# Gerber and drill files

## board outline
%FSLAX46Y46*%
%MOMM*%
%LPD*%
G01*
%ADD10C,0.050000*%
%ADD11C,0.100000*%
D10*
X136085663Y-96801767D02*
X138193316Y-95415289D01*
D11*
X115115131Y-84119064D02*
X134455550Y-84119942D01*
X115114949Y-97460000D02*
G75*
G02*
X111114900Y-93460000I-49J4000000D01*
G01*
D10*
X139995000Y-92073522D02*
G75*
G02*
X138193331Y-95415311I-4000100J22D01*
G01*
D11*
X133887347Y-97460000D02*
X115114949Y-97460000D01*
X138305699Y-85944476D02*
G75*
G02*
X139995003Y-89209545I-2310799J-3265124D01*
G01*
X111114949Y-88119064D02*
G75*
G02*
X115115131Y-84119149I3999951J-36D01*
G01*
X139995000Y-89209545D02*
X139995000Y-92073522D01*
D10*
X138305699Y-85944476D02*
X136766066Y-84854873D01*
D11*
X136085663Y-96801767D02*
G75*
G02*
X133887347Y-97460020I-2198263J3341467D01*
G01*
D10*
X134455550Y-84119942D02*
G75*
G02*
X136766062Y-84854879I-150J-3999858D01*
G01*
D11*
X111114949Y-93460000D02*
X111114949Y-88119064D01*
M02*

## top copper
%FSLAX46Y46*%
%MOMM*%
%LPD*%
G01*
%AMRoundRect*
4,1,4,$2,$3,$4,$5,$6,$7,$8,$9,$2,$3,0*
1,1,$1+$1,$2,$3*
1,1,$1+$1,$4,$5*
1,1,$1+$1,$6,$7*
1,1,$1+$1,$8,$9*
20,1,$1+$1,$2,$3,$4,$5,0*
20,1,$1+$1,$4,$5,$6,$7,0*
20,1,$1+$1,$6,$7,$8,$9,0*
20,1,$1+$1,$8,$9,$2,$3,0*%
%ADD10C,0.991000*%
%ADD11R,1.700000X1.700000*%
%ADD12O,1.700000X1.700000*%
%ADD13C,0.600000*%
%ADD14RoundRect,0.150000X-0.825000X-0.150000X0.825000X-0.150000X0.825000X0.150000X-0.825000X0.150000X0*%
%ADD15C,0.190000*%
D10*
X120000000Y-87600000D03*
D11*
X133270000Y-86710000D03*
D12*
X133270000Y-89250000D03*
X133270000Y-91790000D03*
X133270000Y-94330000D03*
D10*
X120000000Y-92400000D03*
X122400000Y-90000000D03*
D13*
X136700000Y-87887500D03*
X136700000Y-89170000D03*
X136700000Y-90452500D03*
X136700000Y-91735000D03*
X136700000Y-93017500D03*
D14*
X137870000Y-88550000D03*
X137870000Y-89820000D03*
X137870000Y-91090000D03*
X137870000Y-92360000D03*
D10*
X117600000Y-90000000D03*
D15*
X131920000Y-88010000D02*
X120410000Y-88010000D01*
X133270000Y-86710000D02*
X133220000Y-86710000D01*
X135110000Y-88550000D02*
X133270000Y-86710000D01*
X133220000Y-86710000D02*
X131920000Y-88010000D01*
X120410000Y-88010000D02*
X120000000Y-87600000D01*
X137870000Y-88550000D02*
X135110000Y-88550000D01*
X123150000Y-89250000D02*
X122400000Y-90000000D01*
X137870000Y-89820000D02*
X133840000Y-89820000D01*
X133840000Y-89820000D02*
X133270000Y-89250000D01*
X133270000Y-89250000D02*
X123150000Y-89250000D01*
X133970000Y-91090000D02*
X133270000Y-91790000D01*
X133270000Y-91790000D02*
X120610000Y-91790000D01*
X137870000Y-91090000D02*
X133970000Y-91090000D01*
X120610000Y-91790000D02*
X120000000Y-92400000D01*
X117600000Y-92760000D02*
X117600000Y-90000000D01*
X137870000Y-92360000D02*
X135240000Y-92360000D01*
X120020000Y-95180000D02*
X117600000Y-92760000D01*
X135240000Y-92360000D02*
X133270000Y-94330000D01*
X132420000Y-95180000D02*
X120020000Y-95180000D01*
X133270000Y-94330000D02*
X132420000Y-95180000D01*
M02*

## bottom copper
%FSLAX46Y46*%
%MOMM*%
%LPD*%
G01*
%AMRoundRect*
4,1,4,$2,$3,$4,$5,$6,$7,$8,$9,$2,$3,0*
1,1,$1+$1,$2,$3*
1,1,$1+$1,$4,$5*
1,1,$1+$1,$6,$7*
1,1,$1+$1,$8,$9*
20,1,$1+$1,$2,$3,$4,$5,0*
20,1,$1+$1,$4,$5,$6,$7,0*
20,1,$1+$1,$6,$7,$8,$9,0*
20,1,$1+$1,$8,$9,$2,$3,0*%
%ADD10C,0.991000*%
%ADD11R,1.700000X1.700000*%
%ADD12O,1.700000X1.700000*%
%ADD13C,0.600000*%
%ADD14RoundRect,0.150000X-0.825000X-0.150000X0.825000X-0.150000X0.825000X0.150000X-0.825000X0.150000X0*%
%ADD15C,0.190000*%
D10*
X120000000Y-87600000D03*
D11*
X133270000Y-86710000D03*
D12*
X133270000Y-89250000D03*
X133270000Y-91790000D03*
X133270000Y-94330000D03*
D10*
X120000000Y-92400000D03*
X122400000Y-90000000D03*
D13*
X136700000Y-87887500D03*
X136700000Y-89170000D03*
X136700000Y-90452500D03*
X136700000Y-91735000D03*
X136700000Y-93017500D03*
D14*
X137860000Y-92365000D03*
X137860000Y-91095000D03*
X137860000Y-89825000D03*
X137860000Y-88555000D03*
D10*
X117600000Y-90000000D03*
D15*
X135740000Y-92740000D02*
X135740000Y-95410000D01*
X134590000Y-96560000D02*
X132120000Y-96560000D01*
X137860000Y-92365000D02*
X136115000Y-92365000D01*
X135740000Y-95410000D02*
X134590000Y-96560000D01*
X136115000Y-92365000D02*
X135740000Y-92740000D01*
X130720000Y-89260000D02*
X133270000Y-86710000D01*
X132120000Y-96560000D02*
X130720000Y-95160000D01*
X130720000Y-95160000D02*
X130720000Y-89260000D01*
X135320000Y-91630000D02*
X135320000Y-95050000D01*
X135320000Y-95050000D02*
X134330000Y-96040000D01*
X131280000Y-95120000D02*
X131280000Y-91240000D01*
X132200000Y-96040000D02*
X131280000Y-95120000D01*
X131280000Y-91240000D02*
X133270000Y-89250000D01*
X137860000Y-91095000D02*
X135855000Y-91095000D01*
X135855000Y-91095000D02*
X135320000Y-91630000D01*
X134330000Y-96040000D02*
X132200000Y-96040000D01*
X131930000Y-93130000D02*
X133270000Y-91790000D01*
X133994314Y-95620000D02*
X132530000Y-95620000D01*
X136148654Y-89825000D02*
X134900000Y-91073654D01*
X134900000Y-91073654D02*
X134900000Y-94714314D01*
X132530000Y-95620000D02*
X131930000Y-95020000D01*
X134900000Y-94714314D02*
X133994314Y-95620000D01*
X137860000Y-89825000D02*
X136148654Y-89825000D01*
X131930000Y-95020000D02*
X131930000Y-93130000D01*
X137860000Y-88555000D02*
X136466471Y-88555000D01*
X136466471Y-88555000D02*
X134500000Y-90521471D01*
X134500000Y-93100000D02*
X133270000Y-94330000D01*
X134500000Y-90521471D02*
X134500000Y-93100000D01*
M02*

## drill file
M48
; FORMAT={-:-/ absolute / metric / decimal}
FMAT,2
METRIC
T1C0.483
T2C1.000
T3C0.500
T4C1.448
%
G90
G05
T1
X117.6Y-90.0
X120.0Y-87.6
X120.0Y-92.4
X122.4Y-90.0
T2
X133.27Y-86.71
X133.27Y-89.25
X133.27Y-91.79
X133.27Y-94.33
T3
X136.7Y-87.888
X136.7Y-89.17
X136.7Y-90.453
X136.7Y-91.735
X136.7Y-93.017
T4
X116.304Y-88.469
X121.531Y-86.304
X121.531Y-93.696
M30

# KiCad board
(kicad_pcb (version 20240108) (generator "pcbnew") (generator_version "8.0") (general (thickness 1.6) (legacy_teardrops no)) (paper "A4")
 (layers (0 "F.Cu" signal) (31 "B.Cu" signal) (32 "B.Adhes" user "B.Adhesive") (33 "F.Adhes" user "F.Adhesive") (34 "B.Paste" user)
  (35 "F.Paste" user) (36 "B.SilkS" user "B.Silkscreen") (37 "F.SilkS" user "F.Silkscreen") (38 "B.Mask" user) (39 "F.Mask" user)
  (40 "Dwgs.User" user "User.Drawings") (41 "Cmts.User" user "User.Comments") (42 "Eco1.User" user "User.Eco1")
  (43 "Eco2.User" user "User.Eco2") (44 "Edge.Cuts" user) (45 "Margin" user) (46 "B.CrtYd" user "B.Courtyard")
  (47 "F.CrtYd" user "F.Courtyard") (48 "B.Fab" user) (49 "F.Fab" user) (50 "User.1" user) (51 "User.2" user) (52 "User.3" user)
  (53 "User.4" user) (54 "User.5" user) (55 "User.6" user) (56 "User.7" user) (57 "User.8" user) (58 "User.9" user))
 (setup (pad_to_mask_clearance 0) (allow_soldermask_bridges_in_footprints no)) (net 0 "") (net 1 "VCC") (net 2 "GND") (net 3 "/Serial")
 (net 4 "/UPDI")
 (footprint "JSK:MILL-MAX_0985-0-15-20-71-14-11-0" (layer "F.Cu") (at 120 87.6)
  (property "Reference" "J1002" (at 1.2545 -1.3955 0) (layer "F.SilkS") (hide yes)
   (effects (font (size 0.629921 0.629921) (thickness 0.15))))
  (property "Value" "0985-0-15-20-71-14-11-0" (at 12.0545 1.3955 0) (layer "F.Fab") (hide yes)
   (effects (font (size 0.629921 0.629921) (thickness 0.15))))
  (pad "1" thru_hole circle (at 0 0) (size 0.991 0.991) (drill 0.483) (layers "*.Cu" "*.Mask") (remove_unused_layers no) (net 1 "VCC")
   (solder_mask_margin 0.102)))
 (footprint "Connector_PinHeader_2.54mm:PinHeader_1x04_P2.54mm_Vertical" (layer "F.Cu") (at 133.27 86.71)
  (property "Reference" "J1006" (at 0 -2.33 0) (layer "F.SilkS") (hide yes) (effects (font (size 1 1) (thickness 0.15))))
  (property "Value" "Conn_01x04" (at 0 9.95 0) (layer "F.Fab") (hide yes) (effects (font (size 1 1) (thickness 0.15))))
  (pad "1" thru_hole rect (at 0 0) (size 1.7 1.7) (drill 1) (layers "*.Cu" "*.Mask") (remove_unused_layers no) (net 1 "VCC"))
  (pad "2" thru_hole oval (at 0 2.54) (size 1.7 1.7) (drill 1) (layers "*.Cu" "*.Mask") (remove_unused_layers no) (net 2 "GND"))
  (pad "3" thru_hole oval (at 0 5.08) (size 1.7 1.7) (drill 1) (layers "*.Cu" "*.Mask") (remove_unused_layers no) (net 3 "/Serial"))
  (pad "4" thru_hole oval (at 0 7.62) (size 1.7 1.7) (drill 1) (layers "*.Cu" "*.Mask") (remove_unused_layers no) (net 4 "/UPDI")))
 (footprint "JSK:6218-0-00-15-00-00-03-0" (layer "F.Cu") (at 121.530733 93.695518)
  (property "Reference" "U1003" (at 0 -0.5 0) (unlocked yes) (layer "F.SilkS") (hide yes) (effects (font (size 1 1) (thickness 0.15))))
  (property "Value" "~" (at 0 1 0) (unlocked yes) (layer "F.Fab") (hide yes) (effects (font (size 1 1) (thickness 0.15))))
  (pad "" np_thru_hole circle (at 0 0) (size 1.648 1.648) (drill 1.448) (layers "*.Mask")))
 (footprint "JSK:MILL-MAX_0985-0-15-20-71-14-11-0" (layer "F.Cu") (at 120 92.4)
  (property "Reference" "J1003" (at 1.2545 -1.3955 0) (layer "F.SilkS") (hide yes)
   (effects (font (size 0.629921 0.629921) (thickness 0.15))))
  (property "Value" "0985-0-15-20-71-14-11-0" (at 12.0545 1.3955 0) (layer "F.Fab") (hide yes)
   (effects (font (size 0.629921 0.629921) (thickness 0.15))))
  (pad "1" thru_hole circle (at 0 0) (size 0.991 0.991) (drill 0.483) (layers "*.Cu" "*.Mask") (remove_unused_layers no) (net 3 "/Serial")
   (solder_mask_margin 0.102)))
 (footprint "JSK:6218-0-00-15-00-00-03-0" (layer "F.Cu") (at 121.530733 86.304481)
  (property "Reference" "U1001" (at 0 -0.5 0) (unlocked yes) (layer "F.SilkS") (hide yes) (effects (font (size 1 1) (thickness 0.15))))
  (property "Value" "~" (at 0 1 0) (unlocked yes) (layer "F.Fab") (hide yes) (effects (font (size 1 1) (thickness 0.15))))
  (pad "" np_thru_hole circle (at 0 0) (size 1.648 1.648) (drill 1.448) (layers "*.Mask")))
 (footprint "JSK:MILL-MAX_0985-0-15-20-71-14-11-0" (layer "F.Cu") (at 122.4 90)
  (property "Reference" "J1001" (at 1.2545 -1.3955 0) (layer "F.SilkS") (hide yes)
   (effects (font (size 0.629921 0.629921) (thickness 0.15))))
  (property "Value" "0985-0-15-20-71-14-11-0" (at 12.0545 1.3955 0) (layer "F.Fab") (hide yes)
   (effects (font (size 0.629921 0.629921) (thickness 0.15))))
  (pad "1" thru_hole circle (at 0 0) (size 0.991 0.991) (drill 0.483) (layers "*.Cu" "*.Mask") (remove_unused_layers no) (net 2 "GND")
   (solder_mask_margin 0.102)))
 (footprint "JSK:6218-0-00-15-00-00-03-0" (layer "F.Cu") (at 116.304481 88.469266)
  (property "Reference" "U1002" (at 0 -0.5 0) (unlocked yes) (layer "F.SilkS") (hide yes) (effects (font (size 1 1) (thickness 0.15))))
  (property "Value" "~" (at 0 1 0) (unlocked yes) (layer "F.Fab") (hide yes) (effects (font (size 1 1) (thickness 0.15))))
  (pad "" np_thru_hole circle (at 0 0) (size 1.648 1.648) (drill 1.448) (layers "*.Mask")))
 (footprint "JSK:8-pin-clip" (layer "F.Cu") (at 137.87 90.455)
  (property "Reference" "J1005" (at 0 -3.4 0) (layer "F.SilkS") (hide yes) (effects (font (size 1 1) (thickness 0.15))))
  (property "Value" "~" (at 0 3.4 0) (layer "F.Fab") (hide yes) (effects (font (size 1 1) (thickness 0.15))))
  (pad "" np_thru_hole circle (at -1.17 -2.5675) (size 0.6 0.6) (drill 0.5) (layers "F&B.Cu"))
  (pad "" np_thru_hole circle (at -1.17 -1.285) (size 0.6 0.6) (drill 0.5) (layers "F&B.Cu"))
  (pad "" np_thru_hole circle (at -1.17 -0.0025) (size 0.6 0.6) (drill 0.5) (layers "F&B.Cu"))
  (pad "" np_thru_hole circle (at -1.17 1.28) (size 0.6 0.6) (drill 0.5) (layers "F&B.Cu"))
  (pad "" np_thru_hole circle (at -1.17 2.5625) (size 0.6 0.6) (drill 0.5) (layers "F&B.Cu"))
  (pad "A1" smd roundrect (at 0 -1.905) (size 1.95 0.6) (layers "F.Cu" "F.Paste" "F.Mask") (roundrect_rratio 0.25) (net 1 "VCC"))
  (pad "A2" smd roundrect (at 0 -0.635) (size 1.95 0.6) (layers "F.Cu" "F.Paste" "F.Mask") (roundrect_rratio 0.25) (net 2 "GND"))
  (pad "A3" smd roundrect (at 0 0.635) (size 1.95 0.6) (layers "F.Cu" "F.Paste" "F.Mask") (roundrect_rratio 0.25) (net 3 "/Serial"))
  (pad "A4" smd roundrect (at 0 1.905) (size 1.95 0.6) (layers "F.Cu" "F.Paste" "F.Mask") (roundrect_rratio 0.25) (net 4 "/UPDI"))
  (pad "B1" smd roundrect (at -0.01 1.91) (size 1.95 0.6) (layers "B.Cu" "B.Paste" "B.Mask") (roundrect_rratio 0.25) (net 1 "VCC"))
  (pad "B2" smd roundrect (at -0.01 0.64) (size 1.95 0.6) (layers "B.Cu" "B.Paste" "B.Mask") (roundrect_rratio 0.25) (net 2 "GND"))
  (pad "B3" smd roundrect (at -0.01 -0.63) (size 1.95 0.6) (layers "B.Cu" "B.Paste" "B.Mask") (roundrect_rratio 0.25) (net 3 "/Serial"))
  (pad "B4" smd roundrect (at -0.01 -1.9) (size 1.95 0.6) (layers "B.Cu" "B.Paste" "B.Mask") (roundrect_rratio 0.25) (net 4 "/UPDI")))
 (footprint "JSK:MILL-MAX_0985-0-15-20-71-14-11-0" (layer "F.Cu") (at 117.6 90)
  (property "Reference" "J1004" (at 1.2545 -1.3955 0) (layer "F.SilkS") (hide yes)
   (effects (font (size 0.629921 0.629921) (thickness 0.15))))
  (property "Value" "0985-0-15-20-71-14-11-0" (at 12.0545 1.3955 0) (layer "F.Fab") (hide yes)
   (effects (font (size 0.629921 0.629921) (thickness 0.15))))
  (pad "1" thru_hole circle (at 0 0) (size 0.991 0.991) (drill 0.483) (layers "*.Cu" "*.Mask") (remove_unused_layers no) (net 4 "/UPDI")
   (solder_mask_margin 0.102)))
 (gr_line (start 136.085663 96.801767) (end 138.193316 95.415289) (stroke (width 0.05) (type default)) (layer "Edge.Cuts"))
 (gr_line (start 115.115131 84.119064) (end 134.45555 84.119942) (stroke (width 0.1) (type default)) (layer "Edge.Cuts"))
 (gr_arc (start 115.114949 97.46) (mid 112.286522 96.288427) (end 111.114949 93.46) (stroke (width 0.1) (type default)) (layer "Edge.Cuts"))
 (gr_arc (start 139.995 92.073522) (mid 139.515877 93.971769) (end 138.193316 95.415289) (stroke (width 0.05) (type default))
  (layer "Edge.Cuts"))
 (gr_line (start 133.887347 97.46) (end 115.114949 97.46) (stroke (width 0.1) (type default)) (layer "Edge.Cuts"))
 (gr_arc (start 138.305699 85.944476) (mid 139.547645 87.37145) (end 139.995 89.209545) (stroke (width 0.1) (type default))
  (layer "Edge.Cuts"))
 (gr_arc (start 111.114949 88.119064) (mid 112.286586 85.290573) (end 115.115131 84.119064) (stroke (width 0.1) (type default))
  (layer "Edge.Cuts"))
 (gr_line (start 139.995 89.209545) (end 139.995 92.073522) (stroke (width 0.1) (type default)) (layer "Edge.Cuts"))
 (gr_line (start 138.305699 85.944476) (end 136.766066 84.854873) (stroke (width 0.05) (type default)) (layer "Edge.Cuts"))
 (gr_arc (start 136.085663 96.801767) (mid 135.034722 97.291922) (end 133.887347 97.46) (stroke (width 0.1) (type default))
  (layer "Edge.Cuts"))
 (gr_arc (start 134.45555 84.119942) (mid 135.667837 84.308121) (end 136.766066 84.854873) (stroke (width 0.05) (type default))
  (layer "Edge.Cuts"))
 (gr_line (start 111.114949 93.46) (end 111.114949 88.119064) (stroke (width 0.1) (type default)) (layer "Edge.Cuts"))
 (segment (start 131.92 88.01) (end 120.41 88.01) (width 0.19) (layer "F.Cu") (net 1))
 (segment (start 133.27 86.71) (end 133.22 86.71) (width 0.19) (layer "F.Cu") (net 1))
 (segment (start 135.11 88.55) (end 133.27 86.71) (width 0.19) (layer "F.Cu") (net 1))
 (segment (start 133.22 86.71) (end 131.92 88.01) (width 0.19) (layer "F.Cu") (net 1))
 (segment (start 120.41 88.01) (end 120 87.6) (width 0.19) (layer "F.Cu") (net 1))
 (segment (start 137.87 88.55) (end 135.11 88.55) (width 0.19) (layer "F.Cu") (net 1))
 (segment (start 135.74 92.74) (end 135.74 95.41) (width 0.19) (layer "B.Cu") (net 1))
 (segment (start 134.59 96.56) (end 132.12 96.56) (width 0.19) (layer "B.Cu") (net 1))
 (segment (start 137.86 92.365) (end 136.115 92.365) (width 0.19) (layer "B.Cu") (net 1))
 (segment (start 135.74 95.41) (end 134.59 96.56) (width 0.19) (layer "B.Cu") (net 1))
 (segment (start 136.115 92.365) (end 135.74 92.74) (width 0.19) (layer "B.Cu") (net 1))
 (segment (start 130.72 89.26) (end 133.27 86.71) (width 0.19) (layer "B.Cu") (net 1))
 (segment (start 132.12 96.56) (end 130.72 95.16) (width 0.19) (layer "B.Cu") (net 1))
 (segment (start 130.72 95.16) (end 130.72 89.26) (width 0.19) (layer "B.Cu") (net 1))
 (segment (start 123.15 89.25) (end 122.4 90) (width 0.19) (layer "F.Cu") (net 2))
 (segment (start 137.87 89.82) (end 133.84 89.82) (width 0.19) (layer "F.Cu") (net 2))
 (segment (start 133.84 89.82) (end 133.27 89.25) (width 0.19) (layer "F.Cu") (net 2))
 (segment (start 133.27 89.25) (end 123.15 89.25) (width 0.19) (layer "F.Cu") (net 2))
 (segment (start 135.32 91.63) (end 135.32 95.05) (width 0.19) (layer "B.Cu") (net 2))
 (segment (start 135.32 95.05) (end 134.33 96.04) (width 0.19) (layer "B.Cu") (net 2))
 (segment (start 131.28 95.12) (end 131.28 91.24) (width 0.19) (layer "B.Cu") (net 2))
 (segment (start 132.2 96.04) (end 131.28 95.12) (width 0.19) (layer "B.Cu") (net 2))
 (segment (start 131.28 91.24) (end 133.27 89.25) (width 0.19) (layer "B.Cu") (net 2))
 (segment (start 137.86 91.095) (end 135.855 91.095) (width 0.19) (layer "B.Cu") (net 2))
 (segment (start 135.855 91.095) (end 135.32 91.63) (width 0.19) (layer "B.Cu") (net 2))
 (segment (start 134.33 96.04) (end 132.2 96.04) (width 0.19) (layer "B.Cu") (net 2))
 (segment (start 133.97 91.09) (end 133.27 91.79) (width 0.19) (layer "F.Cu") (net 3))
 (segment (start 133.27 91.79) (end 120.61 91.79) (width 0.19) (layer "F.Cu") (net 3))
 (segment (start 137.87 91.09) (end 133.97 91.09) (width 0.19) (layer "F.Cu") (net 3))
 (segment (start 120.61 91.79) (end 120 92.4) (width 0.19) (layer "F.Cu") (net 3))
 (segment (start 131.93 93.13) (end 133.27 91.79) (width 0.19) (layer "B.Cu") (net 3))
 (segment (start 133.994314 95.62) (end 132.53 95.62) (width 0.19) (layer "B.Cu") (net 3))
 (segment (start 136.148654 89.825) (end 134.9 91.073654) (width 0.19) (layer "B.Cu") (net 3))
 (segment (start 134.9 91.073654) (end 134.9 94.714314) (width 0.19) (layer "B.Cu") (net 3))
 (segment (start 132.53 95.62) (end 131.93 95.02) (width 0.19) (layer "B.Cu") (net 3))
 (segment (start 134.9 94.714314) (end 133.994314 95.62) (width 0.19) (layer "B.Cu") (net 3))
 (segment (start 137.86 89.825) (end 136.148654 89.825) (width 0.19) (layer "B.Cu") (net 3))
 (segment (start 131.93 95.02) (end 131.93 93.13) (width 0.19) (layer "B.Cu") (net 3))
 (segment (start 117.6 92.76) (end 117.6 90) (width 0.19) (layer "F.Cu") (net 4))
 (segment (start 137.87 92.36) (end 135.24 92.36) (width 0.19) (layer "F.Cu") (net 4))
 (segment (start 120.02 95.18) (end 117.6 92.76) (width 0.19) (layer "F.Cu") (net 4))
 (segment (start 135.24 92.36) (end 133.27 94.33) (width 0.19) (layer "F.Cu") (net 4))
 (segment (start 132.42 95.18) (end 120.02 95.18) (width 0.19) (layer "F.Cu") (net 4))
 (segment (start 133.27 94.33) (end 132.42 95.18) (width 0.19) (layer "F.Cu") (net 4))
 (segment (start 137.86 88.555) (end 136.466471 88.555) (width 0.19) (layer "B.Cu") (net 4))
 (segment (start 136.466471 88.555) (end 134.5 90.521471) (width 0.19) (layer "B.Cu") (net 4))
 (segment (start 134.5 93.1) (end 133.27 94.33) (width 0.19) (layer "B.Cu") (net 4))
 (segment (start 134.5 90.521471) (end 134.5 93.1) (width 0.19) (layer "B.Cu") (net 4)))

